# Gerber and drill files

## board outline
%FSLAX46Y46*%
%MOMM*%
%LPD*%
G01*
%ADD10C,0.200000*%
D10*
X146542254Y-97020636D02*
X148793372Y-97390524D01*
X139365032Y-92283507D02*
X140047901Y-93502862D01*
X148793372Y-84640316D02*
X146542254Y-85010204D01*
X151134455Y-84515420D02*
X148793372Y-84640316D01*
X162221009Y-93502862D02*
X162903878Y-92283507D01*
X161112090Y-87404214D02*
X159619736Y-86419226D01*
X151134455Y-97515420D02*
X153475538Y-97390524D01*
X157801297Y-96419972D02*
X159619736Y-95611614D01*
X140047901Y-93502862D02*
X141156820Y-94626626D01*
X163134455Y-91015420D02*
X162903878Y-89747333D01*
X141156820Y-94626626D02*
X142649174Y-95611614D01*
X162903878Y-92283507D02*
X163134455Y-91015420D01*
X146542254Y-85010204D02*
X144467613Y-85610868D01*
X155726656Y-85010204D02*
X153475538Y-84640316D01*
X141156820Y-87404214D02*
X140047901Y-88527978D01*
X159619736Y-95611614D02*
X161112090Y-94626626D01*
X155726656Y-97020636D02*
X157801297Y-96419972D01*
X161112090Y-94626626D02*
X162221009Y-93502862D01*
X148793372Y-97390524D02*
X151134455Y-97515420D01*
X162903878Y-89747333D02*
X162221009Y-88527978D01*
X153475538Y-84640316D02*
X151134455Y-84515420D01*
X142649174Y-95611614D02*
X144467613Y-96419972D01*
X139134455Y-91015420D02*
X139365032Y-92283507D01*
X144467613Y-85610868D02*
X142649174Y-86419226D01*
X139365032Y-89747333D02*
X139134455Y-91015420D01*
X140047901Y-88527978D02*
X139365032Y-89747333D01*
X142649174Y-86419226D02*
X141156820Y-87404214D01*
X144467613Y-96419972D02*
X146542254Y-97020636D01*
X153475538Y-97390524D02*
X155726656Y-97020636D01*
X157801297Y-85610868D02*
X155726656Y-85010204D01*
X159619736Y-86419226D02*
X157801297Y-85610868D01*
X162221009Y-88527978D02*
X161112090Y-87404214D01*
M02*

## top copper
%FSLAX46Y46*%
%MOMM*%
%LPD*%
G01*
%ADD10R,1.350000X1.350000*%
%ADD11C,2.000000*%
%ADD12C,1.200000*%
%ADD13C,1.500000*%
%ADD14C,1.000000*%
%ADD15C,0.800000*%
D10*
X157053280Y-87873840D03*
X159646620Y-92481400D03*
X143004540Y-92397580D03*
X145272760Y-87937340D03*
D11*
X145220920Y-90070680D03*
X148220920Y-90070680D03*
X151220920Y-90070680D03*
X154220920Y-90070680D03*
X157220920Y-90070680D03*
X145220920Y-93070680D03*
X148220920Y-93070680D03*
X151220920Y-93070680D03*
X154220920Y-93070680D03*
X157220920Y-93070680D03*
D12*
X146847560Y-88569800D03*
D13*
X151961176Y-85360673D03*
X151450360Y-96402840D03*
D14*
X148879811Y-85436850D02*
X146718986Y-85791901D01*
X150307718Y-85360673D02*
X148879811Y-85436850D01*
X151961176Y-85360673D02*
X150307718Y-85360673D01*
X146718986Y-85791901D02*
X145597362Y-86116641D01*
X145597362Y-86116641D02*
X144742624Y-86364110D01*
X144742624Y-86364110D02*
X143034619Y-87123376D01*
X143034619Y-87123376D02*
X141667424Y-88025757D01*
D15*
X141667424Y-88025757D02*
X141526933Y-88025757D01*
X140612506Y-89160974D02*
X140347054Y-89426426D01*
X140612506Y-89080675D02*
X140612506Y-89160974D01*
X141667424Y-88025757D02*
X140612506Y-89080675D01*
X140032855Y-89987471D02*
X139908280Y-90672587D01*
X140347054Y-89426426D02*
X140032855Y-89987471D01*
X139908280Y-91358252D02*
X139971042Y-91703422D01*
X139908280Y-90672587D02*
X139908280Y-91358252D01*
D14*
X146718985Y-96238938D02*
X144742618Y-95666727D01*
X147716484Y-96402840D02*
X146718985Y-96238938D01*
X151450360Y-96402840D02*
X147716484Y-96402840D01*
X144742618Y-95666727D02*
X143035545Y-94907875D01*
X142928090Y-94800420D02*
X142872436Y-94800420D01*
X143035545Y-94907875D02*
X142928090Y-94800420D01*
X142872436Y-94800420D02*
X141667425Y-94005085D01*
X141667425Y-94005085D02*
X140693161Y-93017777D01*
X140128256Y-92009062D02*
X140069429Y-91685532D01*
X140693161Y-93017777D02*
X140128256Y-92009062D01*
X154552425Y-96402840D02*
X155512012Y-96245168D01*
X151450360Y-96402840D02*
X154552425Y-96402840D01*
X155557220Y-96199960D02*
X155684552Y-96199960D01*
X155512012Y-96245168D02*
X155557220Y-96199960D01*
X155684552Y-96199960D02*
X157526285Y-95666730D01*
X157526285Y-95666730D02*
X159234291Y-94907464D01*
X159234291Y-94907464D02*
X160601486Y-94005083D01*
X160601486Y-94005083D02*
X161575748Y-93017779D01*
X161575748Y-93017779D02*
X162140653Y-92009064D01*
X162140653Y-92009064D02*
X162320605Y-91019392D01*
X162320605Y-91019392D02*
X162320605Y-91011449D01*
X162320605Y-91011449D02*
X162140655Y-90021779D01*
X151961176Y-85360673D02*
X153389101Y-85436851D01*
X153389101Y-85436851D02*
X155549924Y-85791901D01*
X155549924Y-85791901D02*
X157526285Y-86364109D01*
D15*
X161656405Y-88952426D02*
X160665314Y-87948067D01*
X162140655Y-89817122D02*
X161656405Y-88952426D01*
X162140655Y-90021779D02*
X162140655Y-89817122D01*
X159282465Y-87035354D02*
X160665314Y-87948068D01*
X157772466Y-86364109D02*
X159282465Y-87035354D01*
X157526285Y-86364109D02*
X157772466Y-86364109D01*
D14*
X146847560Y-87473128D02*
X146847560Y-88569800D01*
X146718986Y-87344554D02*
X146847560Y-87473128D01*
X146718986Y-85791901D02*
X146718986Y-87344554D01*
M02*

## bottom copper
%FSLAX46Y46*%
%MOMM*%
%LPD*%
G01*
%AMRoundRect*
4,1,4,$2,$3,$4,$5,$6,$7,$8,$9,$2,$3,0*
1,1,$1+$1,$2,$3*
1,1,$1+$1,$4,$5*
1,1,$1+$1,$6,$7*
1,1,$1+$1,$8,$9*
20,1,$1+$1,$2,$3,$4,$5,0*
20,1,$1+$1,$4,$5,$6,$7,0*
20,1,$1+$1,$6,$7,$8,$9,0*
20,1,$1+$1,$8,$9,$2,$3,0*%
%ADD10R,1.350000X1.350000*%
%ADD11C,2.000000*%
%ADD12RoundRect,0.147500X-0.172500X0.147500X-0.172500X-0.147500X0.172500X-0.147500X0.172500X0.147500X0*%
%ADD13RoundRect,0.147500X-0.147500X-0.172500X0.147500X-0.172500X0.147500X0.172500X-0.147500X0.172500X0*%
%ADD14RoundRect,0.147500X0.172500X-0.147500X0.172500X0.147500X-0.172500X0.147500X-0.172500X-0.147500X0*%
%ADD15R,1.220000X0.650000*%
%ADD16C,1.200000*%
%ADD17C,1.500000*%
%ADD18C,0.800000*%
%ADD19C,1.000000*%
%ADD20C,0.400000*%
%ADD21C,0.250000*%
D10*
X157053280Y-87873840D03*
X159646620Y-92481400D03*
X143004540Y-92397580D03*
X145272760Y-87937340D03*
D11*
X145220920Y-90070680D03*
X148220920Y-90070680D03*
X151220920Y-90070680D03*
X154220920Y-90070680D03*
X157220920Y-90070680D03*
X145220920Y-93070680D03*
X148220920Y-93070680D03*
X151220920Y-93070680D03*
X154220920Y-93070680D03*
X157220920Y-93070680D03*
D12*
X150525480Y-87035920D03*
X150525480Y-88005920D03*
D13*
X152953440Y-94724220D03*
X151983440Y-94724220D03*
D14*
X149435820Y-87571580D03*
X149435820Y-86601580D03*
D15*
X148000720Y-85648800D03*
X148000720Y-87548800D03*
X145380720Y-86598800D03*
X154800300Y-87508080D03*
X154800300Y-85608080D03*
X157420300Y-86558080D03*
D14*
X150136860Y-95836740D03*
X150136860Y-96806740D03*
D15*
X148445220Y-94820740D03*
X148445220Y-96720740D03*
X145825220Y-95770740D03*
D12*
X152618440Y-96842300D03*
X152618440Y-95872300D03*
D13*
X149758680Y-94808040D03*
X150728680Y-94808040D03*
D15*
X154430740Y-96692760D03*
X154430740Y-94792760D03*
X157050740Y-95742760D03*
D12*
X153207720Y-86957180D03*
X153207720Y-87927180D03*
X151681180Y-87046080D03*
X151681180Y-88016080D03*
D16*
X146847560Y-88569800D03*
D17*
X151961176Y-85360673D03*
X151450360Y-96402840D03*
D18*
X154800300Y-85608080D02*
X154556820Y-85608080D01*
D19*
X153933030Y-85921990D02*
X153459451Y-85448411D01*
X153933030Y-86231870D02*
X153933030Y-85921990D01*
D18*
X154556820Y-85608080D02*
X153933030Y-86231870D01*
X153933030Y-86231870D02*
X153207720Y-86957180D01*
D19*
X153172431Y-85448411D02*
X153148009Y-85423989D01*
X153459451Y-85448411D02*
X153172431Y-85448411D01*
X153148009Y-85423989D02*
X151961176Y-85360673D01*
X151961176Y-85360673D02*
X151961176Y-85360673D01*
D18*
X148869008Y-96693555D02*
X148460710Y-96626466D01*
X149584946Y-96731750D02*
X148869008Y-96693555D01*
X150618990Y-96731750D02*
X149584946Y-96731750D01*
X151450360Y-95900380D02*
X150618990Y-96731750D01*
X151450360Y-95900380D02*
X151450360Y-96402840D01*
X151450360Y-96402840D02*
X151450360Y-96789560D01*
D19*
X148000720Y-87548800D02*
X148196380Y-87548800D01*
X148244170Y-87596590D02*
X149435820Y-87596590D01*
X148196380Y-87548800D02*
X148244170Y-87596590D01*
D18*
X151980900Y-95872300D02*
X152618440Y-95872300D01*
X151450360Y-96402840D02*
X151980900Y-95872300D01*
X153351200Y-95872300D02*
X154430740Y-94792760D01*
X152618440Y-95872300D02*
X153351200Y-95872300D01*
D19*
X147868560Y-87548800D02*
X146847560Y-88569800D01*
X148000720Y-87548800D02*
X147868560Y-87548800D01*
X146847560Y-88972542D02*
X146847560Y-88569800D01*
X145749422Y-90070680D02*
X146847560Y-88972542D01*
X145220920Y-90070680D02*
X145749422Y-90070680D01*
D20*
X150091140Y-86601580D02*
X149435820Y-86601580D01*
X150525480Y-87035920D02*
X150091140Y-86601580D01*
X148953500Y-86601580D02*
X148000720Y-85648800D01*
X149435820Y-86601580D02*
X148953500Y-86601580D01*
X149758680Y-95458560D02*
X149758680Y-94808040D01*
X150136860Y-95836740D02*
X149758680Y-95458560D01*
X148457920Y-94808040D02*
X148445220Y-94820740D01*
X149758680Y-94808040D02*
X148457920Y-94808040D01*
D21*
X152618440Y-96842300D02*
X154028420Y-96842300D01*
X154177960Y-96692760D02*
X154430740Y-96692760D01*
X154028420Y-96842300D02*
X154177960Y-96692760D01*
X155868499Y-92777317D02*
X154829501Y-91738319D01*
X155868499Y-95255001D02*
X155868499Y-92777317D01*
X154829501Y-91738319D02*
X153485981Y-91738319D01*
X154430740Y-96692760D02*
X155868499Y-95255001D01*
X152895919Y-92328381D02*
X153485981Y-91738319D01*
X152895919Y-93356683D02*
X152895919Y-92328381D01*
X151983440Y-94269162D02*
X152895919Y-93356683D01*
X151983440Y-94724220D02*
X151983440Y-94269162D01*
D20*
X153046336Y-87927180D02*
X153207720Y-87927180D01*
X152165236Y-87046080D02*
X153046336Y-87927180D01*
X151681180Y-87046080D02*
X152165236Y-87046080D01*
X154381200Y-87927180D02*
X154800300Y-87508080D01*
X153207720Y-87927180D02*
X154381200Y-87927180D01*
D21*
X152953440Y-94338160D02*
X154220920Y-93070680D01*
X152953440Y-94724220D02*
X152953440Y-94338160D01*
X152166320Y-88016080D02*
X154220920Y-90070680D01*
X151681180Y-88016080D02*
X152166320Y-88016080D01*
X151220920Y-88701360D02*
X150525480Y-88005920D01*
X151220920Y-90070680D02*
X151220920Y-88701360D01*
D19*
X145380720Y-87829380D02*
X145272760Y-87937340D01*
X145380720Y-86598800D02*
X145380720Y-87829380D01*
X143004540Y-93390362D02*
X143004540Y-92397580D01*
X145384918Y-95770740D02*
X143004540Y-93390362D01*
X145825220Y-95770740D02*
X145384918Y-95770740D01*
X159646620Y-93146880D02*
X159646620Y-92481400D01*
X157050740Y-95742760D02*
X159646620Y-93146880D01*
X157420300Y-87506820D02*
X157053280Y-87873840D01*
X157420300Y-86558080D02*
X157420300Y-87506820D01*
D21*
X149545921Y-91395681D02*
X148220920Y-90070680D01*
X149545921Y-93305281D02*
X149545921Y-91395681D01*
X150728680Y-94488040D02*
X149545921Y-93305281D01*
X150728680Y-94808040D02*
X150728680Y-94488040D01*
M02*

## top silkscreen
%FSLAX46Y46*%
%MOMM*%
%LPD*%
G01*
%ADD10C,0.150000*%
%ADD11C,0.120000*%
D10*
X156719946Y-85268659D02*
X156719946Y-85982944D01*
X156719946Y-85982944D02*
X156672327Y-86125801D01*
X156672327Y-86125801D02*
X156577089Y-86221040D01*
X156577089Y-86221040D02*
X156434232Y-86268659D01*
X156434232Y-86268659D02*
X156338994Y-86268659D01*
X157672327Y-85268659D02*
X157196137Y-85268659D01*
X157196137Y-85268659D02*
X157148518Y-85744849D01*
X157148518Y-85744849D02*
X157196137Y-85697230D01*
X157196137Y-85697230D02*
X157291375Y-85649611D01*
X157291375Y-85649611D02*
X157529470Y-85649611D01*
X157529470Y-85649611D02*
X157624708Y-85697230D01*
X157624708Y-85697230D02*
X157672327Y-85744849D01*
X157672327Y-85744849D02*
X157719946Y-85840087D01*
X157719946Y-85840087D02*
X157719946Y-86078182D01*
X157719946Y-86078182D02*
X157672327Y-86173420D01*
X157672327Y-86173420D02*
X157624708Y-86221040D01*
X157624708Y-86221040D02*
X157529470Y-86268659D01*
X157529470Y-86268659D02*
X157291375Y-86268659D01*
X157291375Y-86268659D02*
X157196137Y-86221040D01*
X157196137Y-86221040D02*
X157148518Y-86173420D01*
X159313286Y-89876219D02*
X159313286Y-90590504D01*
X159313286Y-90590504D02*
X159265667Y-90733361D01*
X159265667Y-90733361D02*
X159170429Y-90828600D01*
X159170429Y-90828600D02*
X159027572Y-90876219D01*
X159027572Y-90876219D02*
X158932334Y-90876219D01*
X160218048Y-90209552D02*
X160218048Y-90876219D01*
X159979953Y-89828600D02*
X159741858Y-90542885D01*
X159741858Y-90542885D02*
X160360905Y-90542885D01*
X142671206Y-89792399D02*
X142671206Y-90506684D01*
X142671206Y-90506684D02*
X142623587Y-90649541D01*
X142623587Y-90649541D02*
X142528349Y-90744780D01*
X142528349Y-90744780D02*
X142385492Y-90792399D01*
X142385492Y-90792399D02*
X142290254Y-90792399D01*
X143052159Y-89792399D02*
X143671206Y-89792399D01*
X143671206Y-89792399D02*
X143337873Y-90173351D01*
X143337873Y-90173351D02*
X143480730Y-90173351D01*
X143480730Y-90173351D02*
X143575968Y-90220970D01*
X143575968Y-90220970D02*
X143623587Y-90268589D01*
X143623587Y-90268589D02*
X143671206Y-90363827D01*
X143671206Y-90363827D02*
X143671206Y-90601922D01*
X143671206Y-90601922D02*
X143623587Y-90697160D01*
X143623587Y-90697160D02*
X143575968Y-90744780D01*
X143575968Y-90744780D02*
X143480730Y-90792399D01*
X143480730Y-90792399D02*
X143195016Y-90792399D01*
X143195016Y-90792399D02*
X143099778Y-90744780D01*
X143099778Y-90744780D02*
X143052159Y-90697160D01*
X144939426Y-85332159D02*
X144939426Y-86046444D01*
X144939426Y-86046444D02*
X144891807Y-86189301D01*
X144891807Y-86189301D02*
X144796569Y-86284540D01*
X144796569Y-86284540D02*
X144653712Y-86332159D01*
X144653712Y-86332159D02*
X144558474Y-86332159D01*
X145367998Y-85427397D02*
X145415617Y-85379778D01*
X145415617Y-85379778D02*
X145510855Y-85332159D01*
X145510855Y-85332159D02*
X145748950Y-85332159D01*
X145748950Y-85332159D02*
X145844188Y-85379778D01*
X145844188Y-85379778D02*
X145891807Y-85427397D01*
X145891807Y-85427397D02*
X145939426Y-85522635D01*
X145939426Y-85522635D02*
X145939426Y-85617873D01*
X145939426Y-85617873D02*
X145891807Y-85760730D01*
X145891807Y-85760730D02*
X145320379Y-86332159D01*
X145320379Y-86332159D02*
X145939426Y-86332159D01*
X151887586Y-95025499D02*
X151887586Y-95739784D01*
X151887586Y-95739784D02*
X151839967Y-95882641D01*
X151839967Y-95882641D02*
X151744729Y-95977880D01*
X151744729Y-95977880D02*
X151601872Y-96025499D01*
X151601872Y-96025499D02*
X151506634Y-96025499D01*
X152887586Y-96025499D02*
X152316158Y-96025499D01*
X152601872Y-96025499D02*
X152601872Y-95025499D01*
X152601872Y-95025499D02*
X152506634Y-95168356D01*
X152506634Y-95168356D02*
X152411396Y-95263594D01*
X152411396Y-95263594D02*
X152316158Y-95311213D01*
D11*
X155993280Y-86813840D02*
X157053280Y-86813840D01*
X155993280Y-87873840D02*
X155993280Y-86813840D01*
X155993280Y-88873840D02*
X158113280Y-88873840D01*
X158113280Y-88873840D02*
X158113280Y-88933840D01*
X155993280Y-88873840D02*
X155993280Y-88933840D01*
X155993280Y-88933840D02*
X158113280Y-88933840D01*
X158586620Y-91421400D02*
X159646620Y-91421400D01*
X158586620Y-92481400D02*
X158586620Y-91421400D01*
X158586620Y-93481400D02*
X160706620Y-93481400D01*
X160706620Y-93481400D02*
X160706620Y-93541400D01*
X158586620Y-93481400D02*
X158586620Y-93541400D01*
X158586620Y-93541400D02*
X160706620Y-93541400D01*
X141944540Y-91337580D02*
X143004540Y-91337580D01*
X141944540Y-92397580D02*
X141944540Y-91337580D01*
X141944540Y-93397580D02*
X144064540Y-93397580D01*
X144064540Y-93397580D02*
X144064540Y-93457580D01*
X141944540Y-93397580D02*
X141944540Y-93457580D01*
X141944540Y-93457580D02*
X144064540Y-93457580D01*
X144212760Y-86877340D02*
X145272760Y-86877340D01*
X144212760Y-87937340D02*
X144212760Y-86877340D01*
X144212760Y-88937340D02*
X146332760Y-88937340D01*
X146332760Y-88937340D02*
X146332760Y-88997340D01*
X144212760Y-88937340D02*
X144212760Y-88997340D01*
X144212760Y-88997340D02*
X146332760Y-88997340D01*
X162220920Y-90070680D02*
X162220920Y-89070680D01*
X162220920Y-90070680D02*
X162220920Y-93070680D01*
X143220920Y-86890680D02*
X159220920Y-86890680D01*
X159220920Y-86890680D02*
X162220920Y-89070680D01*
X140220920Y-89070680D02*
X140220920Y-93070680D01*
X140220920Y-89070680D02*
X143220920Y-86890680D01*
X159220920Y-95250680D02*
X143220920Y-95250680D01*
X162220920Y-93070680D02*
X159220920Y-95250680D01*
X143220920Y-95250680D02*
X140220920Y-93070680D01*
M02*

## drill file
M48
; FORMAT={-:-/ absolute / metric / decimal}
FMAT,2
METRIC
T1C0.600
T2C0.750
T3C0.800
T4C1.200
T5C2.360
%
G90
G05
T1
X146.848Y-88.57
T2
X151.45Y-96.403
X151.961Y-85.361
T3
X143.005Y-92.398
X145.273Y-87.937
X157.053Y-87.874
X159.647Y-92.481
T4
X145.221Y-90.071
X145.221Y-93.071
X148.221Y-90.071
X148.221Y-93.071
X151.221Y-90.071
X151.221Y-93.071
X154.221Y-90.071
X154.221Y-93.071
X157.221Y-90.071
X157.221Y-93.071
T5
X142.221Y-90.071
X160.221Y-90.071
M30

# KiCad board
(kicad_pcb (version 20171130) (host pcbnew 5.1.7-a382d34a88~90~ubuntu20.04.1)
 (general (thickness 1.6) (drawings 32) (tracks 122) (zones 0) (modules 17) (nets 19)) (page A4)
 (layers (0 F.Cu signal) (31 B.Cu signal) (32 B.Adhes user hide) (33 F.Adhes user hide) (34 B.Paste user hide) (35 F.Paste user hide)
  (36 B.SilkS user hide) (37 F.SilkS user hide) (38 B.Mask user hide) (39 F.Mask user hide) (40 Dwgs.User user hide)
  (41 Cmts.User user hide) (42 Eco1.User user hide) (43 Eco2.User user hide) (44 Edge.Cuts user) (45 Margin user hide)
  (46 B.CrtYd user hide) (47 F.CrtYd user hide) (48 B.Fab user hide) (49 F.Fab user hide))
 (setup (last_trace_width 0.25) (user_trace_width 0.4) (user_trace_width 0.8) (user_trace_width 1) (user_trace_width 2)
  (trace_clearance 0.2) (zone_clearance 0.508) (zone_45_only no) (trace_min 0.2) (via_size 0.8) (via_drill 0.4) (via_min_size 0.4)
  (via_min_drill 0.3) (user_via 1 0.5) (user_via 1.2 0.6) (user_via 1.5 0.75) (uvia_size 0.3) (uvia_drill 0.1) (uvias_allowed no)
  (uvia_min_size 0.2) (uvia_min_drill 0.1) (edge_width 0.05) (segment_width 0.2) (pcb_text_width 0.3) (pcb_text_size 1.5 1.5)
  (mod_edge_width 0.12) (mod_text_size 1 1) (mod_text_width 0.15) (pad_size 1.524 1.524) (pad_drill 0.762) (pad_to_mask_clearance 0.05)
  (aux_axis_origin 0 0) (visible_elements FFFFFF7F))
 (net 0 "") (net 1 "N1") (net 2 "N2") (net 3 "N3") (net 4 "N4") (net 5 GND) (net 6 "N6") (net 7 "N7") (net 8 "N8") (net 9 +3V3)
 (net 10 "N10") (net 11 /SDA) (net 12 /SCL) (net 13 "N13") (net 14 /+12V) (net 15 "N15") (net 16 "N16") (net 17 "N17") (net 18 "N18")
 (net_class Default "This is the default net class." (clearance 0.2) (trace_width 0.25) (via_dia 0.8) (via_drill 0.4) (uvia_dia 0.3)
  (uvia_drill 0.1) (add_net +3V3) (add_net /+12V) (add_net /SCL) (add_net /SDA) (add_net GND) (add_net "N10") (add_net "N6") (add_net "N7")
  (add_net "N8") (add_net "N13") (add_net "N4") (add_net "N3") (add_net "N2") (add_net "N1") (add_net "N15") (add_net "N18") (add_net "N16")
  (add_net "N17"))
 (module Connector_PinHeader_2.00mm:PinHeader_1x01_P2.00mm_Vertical (layer F.Cu) (at 157.05328 87.87384)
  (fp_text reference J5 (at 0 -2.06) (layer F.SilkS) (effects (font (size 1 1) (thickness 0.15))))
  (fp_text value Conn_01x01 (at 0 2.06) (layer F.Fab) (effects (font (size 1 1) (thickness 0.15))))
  (fp_line (start -1.06 -1.06) (end 0 -1.06) (layer F.SilkS) (width 0.12))
  (fp_line (start -1.06 0) (end -1.06 -1.06) (layer F.SilkS) (width 0.12))
  (fp_line (start -1.06 1) (end 1.06 1) (layer F.SilkS) (width 0.12))
  (fp_line (start 1.06 1) (end 1.06 1.06) (layer F.SilkS) (width 0.12))
  (fp_line (start -1.06 1) (end -1.06 1.06) (layer F.SilkS) (width 0.12))
  (fp_line (start -1.06 1.06) (end 1.06 1.06) (layer F.SilkS) (width 0.12))
  (pad 1 thru_hole rect (at 0 0) (size 1.35 1.35) (drill 0.8) (layers *.Cu *.Mask) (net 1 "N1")))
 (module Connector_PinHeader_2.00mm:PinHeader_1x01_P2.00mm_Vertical (layer F.Cu) (at 159.64662 92.4814)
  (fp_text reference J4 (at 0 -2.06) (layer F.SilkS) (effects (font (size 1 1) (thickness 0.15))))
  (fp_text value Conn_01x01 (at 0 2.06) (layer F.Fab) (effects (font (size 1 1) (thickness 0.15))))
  (fp_line (start -1.06 -1.06) (end 0 -1.06) (layer F.SilkS) (width 0.12))
  (fp_line (start -1.06 0) (end -1.06 -1.06) (layer F.SilkS) (width 0.12))
  (fp_line (start -1.06 1) (end 1.06 1) (layer F.SilkS) (width 0.12))
  (fp_line (start 1.06 1) (end 1.06 1.06) (layer F.SilkS) (width 0.12))
  (fp_line (start -1.06 1) (end -1.06 1.06) (layer F.SilkS) (width 0.12))
  (fp_line (start -1.06 1.06) (end 1.06 1.06) (layer F.SilkS) (width 0.12))
  (pad 1 thru_hole rect (at 0 0) (size 1.35 1.35) (drill 0.8) (layers *.Cu *.Mask) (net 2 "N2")))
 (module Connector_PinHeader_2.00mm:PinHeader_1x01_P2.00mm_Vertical (layer F.Cu) (at 143.00454 92.39758)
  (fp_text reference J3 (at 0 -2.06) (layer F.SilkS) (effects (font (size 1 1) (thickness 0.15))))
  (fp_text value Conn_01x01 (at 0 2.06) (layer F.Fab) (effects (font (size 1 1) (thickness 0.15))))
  (fp_line (start -1.06 -1.06) (end 0 -1.06) (layer F.SilkS) (width 0.12))
  (fp_line (start -1.06 0) (end -1.06 -1.06) (layer F.SilkS) (width 0.12))
  (fp_line (start -1.06 1) (end 1.06 1) (layer F.SilkS) (width 0.12))
  (fp_line (start 1.06 1) (end 1.06 1.06) (layer F.SilkS) (width 0.12))
  (fp_line (start -1.06 1) (end -1.06 1.06) (layer F.SilkS) (width 0.12))
  (fp_line (start -1.06 1.06) (end 1.06 1.06) (layer F.SilkS) (width 0.12))
  (pad 1 thru_hole rect (at 0 0) (size 1.35 1.35) (drill 0.8) (layers *.Cu *.Mask) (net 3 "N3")))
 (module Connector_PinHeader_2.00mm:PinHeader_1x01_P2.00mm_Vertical (layer F.Cu) (at 145.27276 87.93734)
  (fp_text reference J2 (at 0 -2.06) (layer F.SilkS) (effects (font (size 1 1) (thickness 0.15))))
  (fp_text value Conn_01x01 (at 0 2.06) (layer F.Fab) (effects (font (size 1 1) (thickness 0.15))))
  (fp_line (start -1.06 -1.06) (end 0 -1.06) (layer F.SilkS) (width 0.12))
  (fp_line (start -1.06 0) (end -1.06 -1.06) (layer F.SilkS) (width 0.12))
  (fp_line (start -1.06 1) (end 1.06 1) (layer F.SilkS) (width 0.12))
  (fp_line (start 1.06 1) (end 1.06 1.06) (layer F.SilkS) (width 0.12))
  (fp_line (start -1.06 1) (end -1.06 1.06) (layer F.SilkS) (width 0.12))
  (fp_line (start -1.06 1.06) (end 1.06 1.06) (layer F.SilkS) (width 0.12))
  (pad 1 thru_hole rect (at 0 0) (size 1.35 1.35) (drill 0.8) (layers *.Cu *.Mask) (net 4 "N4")))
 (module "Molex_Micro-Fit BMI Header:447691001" (layer F.Cu) (at 152.22092 95.07068)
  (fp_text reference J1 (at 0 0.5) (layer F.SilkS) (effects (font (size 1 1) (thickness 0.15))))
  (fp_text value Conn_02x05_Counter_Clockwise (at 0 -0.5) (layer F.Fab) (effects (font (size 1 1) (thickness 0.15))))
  (fp_line (start 10 -5) (end 10 -6) (layer F.SilkS) (width 0.12))
  (fp_line (start 10 -5) (end 10 -2) (layer F.SilkS) (width 0.12))
  (fp_line (start -9 -8.18) (end 7 -8.18) (layer F.SilkS) (width 0.12))
  (fp_line (start 7 -8.18) (end 10 -6) (layer F.SilkS) (width 0.12))
  (fp_line (start -12 -6) (end -12 -2) (layer F.SilkS) (width 0.12))
  (fp_line (start -12 -6) (end -9 -8.18) (layer F.SilkS) (width 0.12))
  (fp_line (start 7 0.18) (end -9 0.18) (layer F.SilkS) (width 0.12))
  (fp_line (start 10 -2) (end 7 0.18) (layer F.SilkS) (width 0.12))
  (fp_line (start -9 0.18) (end -12 -2) (layer F.SilkS) (width 0.12))
  (pad "" np_thru_hole circle (at -10 -5) (size 2.36 2.36) (drill 2.36) (layers *.Cu *.Mask))
  (pad "" np_thru_hole circle (at 8 -5) (size 2.36 2.36) (drill 2.36) (layers *.Cu *.Mask))
  (pad 1 thru_hole circle (at -7 -5) (size 2 2) (drill 1.2) (layers *.Cu *.Mask) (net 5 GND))
  (pad 3 thru_hole circle (at -4 -5) (size 2 2) (drill 1.2) (layers *.Cu *.Mask) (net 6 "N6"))
  (pad 5 thru_hole circle (at -1 -5) (size 2 2) (drill 1.2) (layers *.Cu *.Mask) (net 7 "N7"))
  (pad 7 thru_hole circle (at 2 -5) (size 2 2) (drill 1.2) (layers *.Cu *.Mask) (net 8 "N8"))
  (pad 9 thru_hole circle (at 5 -5) (size 2 2) (drill 1.2) (layers *.Cu *.Mask) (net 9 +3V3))
  (pad 2 thru_hole circle (at -7 -2) (size 2 2) (drill 1.2) (layers *.Cu *.Mask) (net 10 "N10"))
  (pad 4 thru_hole circle (at -4 -2) (size 2 2) (drill 1.2) (layers *.Cu *.Mask) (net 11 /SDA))
  (pad 6 thru_hole circle (at -1 -2) (size 2 2) (drill 1.2) (layers *.Cu *.Mask) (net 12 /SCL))
  (pad 8 thru_hole circle (at 2 -2) (size 2 2) (drill 1.2) (layers *.Cu *.Mask) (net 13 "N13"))
  (pad 10 thru_hole circle (at 5 -2) (size 2 2) (drill 1.2) (layers *.Cu *.Mask) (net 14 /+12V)))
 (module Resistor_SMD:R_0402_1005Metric (layer B.Cu) (at 150.52548 87.52092 270)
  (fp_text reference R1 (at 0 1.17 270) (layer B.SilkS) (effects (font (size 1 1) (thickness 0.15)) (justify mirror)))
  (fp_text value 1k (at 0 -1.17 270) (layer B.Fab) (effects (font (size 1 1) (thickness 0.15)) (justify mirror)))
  (pad 1 smd roundrect (at -0.485 0 270) (size 0.59 0.64) (layers B.Cu B.Paste B.Mask) (roundrect_rratio 0.25) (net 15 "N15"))
  (pad 2 smd roundrect (at 0.485 0 270) (size 0.59 0.64) (layers B.Cu B.Paste B.Mask) (roundrect_rratio 0.25) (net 7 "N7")))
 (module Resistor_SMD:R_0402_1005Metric (layer B.Cu) (at 152.46844 94.72422)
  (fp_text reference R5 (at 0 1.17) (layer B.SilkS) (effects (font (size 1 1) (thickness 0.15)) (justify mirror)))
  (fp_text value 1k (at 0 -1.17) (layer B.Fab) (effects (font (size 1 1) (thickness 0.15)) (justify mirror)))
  (pad 2 smd roundrect (at 0.485 0) (size 0.59 0.64) (layers B.Cu B.Paste B.Mask) (roundrect_rratio 0.25) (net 13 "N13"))
  (pad 1 smd roundrect (at -0.485 0) (size 0.59 0.64) (layers B.Cu B.Paste B.Mask) (roundrect_rratio 0.25) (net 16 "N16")))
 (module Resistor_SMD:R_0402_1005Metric (layer B.Cu) (at 149.43582 87.08658 90)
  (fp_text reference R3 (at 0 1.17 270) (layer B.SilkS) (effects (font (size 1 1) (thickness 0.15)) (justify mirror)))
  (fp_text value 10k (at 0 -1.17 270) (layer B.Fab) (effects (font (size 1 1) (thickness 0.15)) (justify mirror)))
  (pad 1 smd roundrect (at -0.485 0 90) (size 0.59 0.64) (layers B.Cu B.Paste B.Mask) (roundrect_rratio 0.25) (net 5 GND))
  (pad 2 smd roundrect (at 0.485 0 90) (size 0.59 0.64) (layers B.Cu B.Paste B.Mask) (roundrect_rratio 0.25) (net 15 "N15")))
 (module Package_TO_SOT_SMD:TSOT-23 (layer B.Cu) (at 146.69072 86.5988 180)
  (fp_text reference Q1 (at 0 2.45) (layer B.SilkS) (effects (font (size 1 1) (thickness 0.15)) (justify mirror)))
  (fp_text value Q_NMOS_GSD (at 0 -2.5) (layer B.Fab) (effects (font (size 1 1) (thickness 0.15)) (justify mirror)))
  (pad 1 smd rect (at -1.31 0.95 180) (size 1.22 0.65) (layers B.Cu B.Paste B.Mask) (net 15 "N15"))
  (pad 2 smd rect (at -1.31 -0.95 180) (size 1.22 0.65) (layers B.Cu B.Paste B.Mask) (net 5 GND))
  (pad 3 smd rect (at 1.31 0 180) (size 1.22 0.65) (layers B.Cu B.Paste B.Mask) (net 4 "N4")))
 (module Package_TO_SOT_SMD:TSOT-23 (layer B.Cu) (at 156.1103 86.55808)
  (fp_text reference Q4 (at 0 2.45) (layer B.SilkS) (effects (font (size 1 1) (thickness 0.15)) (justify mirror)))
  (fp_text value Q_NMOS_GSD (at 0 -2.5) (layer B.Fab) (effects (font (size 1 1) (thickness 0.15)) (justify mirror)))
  (pad 1 smd rect (at -1.31 0.95) (size 1.22 0.65) (layers B.Cu B.Paste B.Mask) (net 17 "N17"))
  (pad 2 smd rect (at -1.31 -0.95) (size 1.22 0.65) (layers B.Cu B.Paste B.Mask) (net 5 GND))
  (pad 3 smd rect (at 1.31 0) (size 1.22 0.65) (layers B.Cu B.Paste B.Mask) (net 1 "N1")))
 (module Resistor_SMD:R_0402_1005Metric (layer B.Cu) (at 150.13686 96.32174 90)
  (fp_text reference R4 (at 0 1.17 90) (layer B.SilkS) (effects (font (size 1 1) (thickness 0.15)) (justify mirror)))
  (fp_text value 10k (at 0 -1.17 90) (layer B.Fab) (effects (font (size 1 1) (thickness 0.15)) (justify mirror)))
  (pad 2 smd roundrect (at 0.485 0 90) (size 0.59 0.64) (layers B.Cu B.Paste B.Mask) (roundrect_rratio 0.25) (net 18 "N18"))
  (pad 1 smd roundrect (at -0.485 0 90) (size 0.59 0.64) (layers B.Cu B.Paste B.Mask) (roundrect_rratio 0.25) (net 5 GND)))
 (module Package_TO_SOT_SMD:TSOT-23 (layer B.Cu) (at 147.13522 95.77074 180)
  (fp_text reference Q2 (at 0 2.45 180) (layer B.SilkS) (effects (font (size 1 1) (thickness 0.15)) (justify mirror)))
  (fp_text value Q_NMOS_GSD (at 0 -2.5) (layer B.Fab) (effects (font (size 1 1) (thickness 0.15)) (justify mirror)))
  (pad 1 smd rect (at -1.31 0.95 180) (size 1.22 0.65) (layers B.Cu B.Paste B.Mask) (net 18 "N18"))
  (pad 2 smd rect (at -1.31 -0.95 180) (size 1.22 0.65) (layers B.Cu B.Paste B.Mask) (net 5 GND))
  (pad 3 smd rect (at 1.31 0 180) (size 1.22 0.65) (layers B.Cu B.Paste B.Mask) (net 3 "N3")))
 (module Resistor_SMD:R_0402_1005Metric (layer B.Cu) (at 152.61844 96.3573 270)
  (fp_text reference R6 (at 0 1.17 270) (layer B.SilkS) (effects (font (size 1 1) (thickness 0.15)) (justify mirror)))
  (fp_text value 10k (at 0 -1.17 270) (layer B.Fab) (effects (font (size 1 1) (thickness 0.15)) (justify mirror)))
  (pad 2 smd roundrect (at 0.485 0 270) (size 0.59 0.64) (layers B.Cu B.Paste B.Mask) (roundrect_rratio 0.25) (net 16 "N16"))
  (pad 1 smd roundrect (at -0.485 0 270) (size 0.59 0.64) (layers B.Cu B.Paste B.Mask) (roundrect_rratio 0.25) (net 5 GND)))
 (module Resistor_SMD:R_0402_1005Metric (layer B.Cu) (at 150.24368 94.80804)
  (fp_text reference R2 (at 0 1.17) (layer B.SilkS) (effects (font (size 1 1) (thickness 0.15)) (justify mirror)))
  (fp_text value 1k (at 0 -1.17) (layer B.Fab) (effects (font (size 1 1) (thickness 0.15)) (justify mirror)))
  (pad 1 smd roundrect (at -0.485 0) (size 0.59 0.64) (layers B.Cu B.Paste B.Mask) (roundrect_rratio 0.25) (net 18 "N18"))
  (pad 2 smd roundrect (at 0.485 0) (size 0.59 0.64) (layers B.Cu B.Paste B.Mask) (roundrect_rratio 0.25) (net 6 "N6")))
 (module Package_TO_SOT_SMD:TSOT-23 (layer B.Cu) (at 155.74074 95.74276)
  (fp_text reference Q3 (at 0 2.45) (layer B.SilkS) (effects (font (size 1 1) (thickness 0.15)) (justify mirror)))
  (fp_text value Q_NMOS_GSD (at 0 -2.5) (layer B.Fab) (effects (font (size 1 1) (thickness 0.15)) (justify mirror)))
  (pad 1 smd rect (at -1.31 0.95) (size 1.22 0.65) (layers B.Cu B.Paste B.Mask) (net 16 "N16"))
  (pad 2 smd rect (at -1.31 -0.95) (size 1.22 0.65) (layers B.Cu B.Paste B.Mask) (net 5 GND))
  (pad 3 smd rect (at 1.31 0) (size 1.22 0.65) (layers B.Cu B.Paste B.Mask) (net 2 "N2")))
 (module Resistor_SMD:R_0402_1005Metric (layer B.Cu) (at 153.20772 87.44218 270)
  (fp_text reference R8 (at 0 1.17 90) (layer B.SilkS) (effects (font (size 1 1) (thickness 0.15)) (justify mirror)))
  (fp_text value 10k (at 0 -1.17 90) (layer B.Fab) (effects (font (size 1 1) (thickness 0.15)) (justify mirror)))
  (pad 1 smd roundrect (at -0.485 0 270) (size 0.59 0.64) (layers B.Cu B.Paste B.Mask) (roundrect_rratio 0.25) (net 5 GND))
  (pad 2 smd roundrect (at 0.485 0 270) (size 0.59 0.64) (layers B.Cu B.Paste B.Mask) (roundrect_rratio 0.25) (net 17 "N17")))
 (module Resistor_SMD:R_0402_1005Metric (layer B.Cu) (at 151.68118 87.53108 270)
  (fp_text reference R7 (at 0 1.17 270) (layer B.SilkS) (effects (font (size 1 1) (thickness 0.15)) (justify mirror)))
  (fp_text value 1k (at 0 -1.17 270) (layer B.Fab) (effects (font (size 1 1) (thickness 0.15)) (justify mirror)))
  (pad 1 smd roundrect (at -0.485 0 270) (size 0.59 0.64) (layers B.Cu B.Paste B.Mask) (roundrect_rratio 0.25) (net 17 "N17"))
  (pad 2 smd roundrect (at 0.485 0 270) (size 0.59 0.64) (layers B.Cu B.Paste B.Mask) (roundrect_rratio 0.25) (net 8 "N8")))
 (gr_line (start 146.542254 97.020636) (end 148.793372 97.390524) (layer Edge.Cuts) (width 0.2))
 (gr_line (start 139.365032 92.283507) (end 140.047901 93.502862) (layer Edge.Cuts) (width 0.2))
 (gr_line (start 148.793372 84.640316) (end 146.542254 85.010204) (layer Edge.Cuts) (width 0.2))
 (gr_line (start 151.134455 84.51542) (end 148.793372 84.640316) (layer Edge.Cuts) (width 0.2))
 (gr_line (start 162.221009 93.502862) (end 162.903878 92.283507) (layer Edge.Cuts) (width 0.2))
 (gr_line (start 161.11209 87.404214) (end 159.619736 86.419226) (layer Edge.Cuts) (width 0.2))
 (gr_line (start 151.134455 97.51542) (end 153.475538 97.390524) (layer Edge.Cuts) (width 0.2))
 (gr_line (start 157.801297 96.419972) (end 159.619736 95.611614) (layer Edge.Cuts) (width 0.2))
 (gr_line (start 140.047901 93.502862) (end 141.15682 94.626626) (layer Edge.Cuts) (width 0.2))
 (gr_line (start 163.134455 91.01542) (end 162.903878 89.747333) (layer Edge.Cuts) (width 0.2))
 (gr_line (start 141.15682 94.626626) (end 142.649174 95.611614) (layer Edge.Cuts) (width 0.2))
 (gr_line (start 162.903878 92.283507) (end 163.134455 91.01542) (layer Edge.Cuts) (width 0.2))
 (gr_line (start 146.542254 85.010204) (end 144.467613 85.610868) (layer Edge.Cuts) (width 0.2))
 (gr_line (start 155.726656 85.010204) (end 153.475538 84.640316) (layer Edge.Cuts) (width 0.2))
 (gr_line (start 141.15682 87.404214) (end 140.047901 88.527978) (layer Edge.Cuts) (width 0.2))
 (gr_line (start 159.619736 95.611614) (end 161.11209 94.626626) (layer Edge.Cuts) (width 0.2))
 (gr_line (start 155.726656 97.020636) (end 157.801297 96.419972) (layer Edge.Cuts) (width 0.2))
 (gr_line (start 161.11209 94.626626) (end 162.221009 93.502862) (layer Edge.Cuts) (width 0.2))
 (gr_line (start 148.793372 97.390524) (end 151.134455 97.51542) (layer Edge.Cuts) (width 0.2))
 (gr_line (start 162.903878 89.747333) (end 162.221009 88.527978) (layer Edge.Cuts) (width 0.2))
 (gr_line (start 153.475538 84.640316) (end 151.134455 84.51542) (layer Edge.Cuts) (width 0.2))
 (gr_line (start 142.649174 95.611614) (end 144.467613 96.419972) (layer Edge.Cuts) (width 0.2))
 (gr_line (start 139.134455 91.01542) (end 139.365032 92.283507) (layer Edge.Cuts) (width 0.2))
 (gr_line (start 144.467613 85.610868) (end 142.649174 86.419226) (layer Edge.Cuts) (width 0.2))
 (gr_line (start 139.365032 89.747333) (end 139.134455 91.01542) (layer Edge.Cuts) (width 0.2))
 (gr_line (start 140.047901 88.527978) (end 139.365032 89.747333) (layer Edge.Cuts) (width 0.2))
 (gr_line (start 142.649174 86.419226) (end 141.15682 87.404214) (layer Edge.Cuts) (width 0.2))
 (gr_line (start 144.467613 96.419972) (end 146.542254 97.020636) (layer Edge.Cuts) (width 0.2))
 (gr_line (start 153.475538 97.390524) (end 155.726656 97.020636) (layer Edge.Cuts) (width 0.2))
 (gr_line (start 157.801297 85.610868) (end 155.726656 85.010204) (layer Edge.Cuts) (width 0.2))
 (gr_line (start 159.619736 86.419226) (end 157.801297 85.610868) (layer Edge.Cuts) (width 0.2))
 (gr_line (start 162.221009 88.527978) (end 161.11209 87.404214) (layer Edge.Cuts) (width 0.2))
 (via (at 146.84756 88.5698) (size 1.2) (drill 0.6) (layers F.Cu B.Cu) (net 5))
 (segment (start 154.8003 85.60808) (end 154.55682 85.60808) (width 0.8) (layer B.Cu) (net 5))
 (segment (start 153.93303 85.92199) (end 153.459451 85.448411) (width 1) (layer B.Cu) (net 5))
 (segment (start 153.93303 86.23187) (end 153.93303 85.92199) (width 1) (layer B.Cu) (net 5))
 (segment (start 154.55682 85.60808) (end 153.93303 86.23187) (width 0.8) (layer B.Cu) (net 5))
 (segment (start 153.93303 86.23187) (end 153.20772 86.95718) (width 0.8) (layer B.Cu) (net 5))
 (segment (start 153.172431 85.448411) (end 153.148009 85.423989) (width 1) (layer B.Cu) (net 5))
 (segment (start 153.459451 85.448411) (end 153.172431 85.448411) (width 1) (layer B.Cu) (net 5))
 (segment (start 153.148009 85.423989) (end 151.961176 85.360673) (width 1) (layer B.Cu) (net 5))
 (segment (start 151.961176 85.360673) (end 151.961176 85.360673) (width 1) (layer B.Cu) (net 5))
 (via (at 151.961176 85.360673) (size 1.5) (drill 0.75) (layers F.Cu B.Cu) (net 5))
 (segment (start 148.879811 85.43685) (end 146.718986 85.791901) (width 1) (layer F.Cu) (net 5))
 (segment (start 150.307718 85.360673) (end 148.879811 85.43685) (width 1) (layer F.Cu) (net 5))
 (segment (start 151.961176 85.360673) (end 150.307718 85.360673) (width 1) (layer F.Cu) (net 5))
 (segment (start 146.718986 85.791901) (end 145.597362 86.116641) (width 1) (layer F.Cu) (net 5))
 (segment (start 145.597362 86.116641) (end 144.742624 86.36411) (width 1) (layer F.Cu) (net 5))
 (segment (start 144.742624 86.36411) (end 143.034619 87.123376) (width 1) (layer F.Cu) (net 5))
 (segment (start 143.034619 87.123376) (end 141.667424 88.025757) (width 1) (layer F.Cu) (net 5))
 (segment (start 141.667424 88.025757) (end 141.526933 88.025757) (width 0.8) (layer F.Cu) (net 5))
 (segment (start 140.612506 89.160974) (end 140.347054 89.426426) (width 0.8) (layer F.Cu) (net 5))
 (segment (start 140.612506 89.080675) (end 140.612506 89.160974) (width 0.8) (layer F.Cu) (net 5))
 (segment (start 141.667424 88.025757) (end 140.612506 89.080675) (width 0.8) (layer F.Cu) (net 5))
 (segment (start 140.032855 89.987471) (end 139.90828 90.672587) (width 0.8) (layer F.Cu) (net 5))
 (segment (start 140.347054 89.426426) (end 140.032855 89.987471) (width 0.8) (layer F.Cu) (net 5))
 (segment (start 139.90828 91.358252) (end 139.971042 91.703422) (width 0.8) (layer F.Cu) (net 5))
 (segment (start 139.90828 90.672587) (end 139.90828 91.358252) (width 0.8) (layer F.Cu) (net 5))
 (segment (start 148.869008 96.693555) (end 148.46071 96.626466) (width 0.8) (layer B.Cu) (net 5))
 (segment (start 149.584946 96.73175) (end 148.869008 96.693555) (width 0.8) (layer B.Cu) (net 5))
 (segment (start 150.61899 96.73175) (end 149.584946 96.73175) (width 0.8) (layer B.Cu) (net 5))
 (segment (start 151.45036 95.90038) (end 150.61899 96.73175) (width 0.8) (layer B.Cu) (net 5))
 (segment (start 151.45036 95.90038) (end 151.45036 96.40284) (width 0.8) (layer B.Cu) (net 5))
 (segment (start 151.45036 96.40284) (end 151.45036 96.78956) (width 0.8) (layer B.Cu) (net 5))
 (via (at 151.45036 96.40284) (size 1.5) (drill 0.75) (layers F.Cu B.Cu) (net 5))
 (segment (start 148.00072 87.5488) (end 148.19638 87.5488) (width 1) (layer B.Cu) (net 5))
 (segment (start 148.24417 87.59659) (end 149.43582 87.59659) (width 1) (layer B.Cu) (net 5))
 (segment (start 148.19638 87.5488) (end 148.24417 87.59659) (width 1) (layer B.Cu) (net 5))
 (segment (start 146.718985 96.238938) (end 144.742618 95.666727) (width 1) (layer F.Cu) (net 5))
 (segment (start 147.716484 96.40284) (end 146.718985 96.238938) (width 1) (layer F.Cu) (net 5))
 (segment (start 151.45036 96.40284) (end 147.716484 96.40284) (width 1) (layer F.Cu) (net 5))
 (segment (start 144.742618 95.666727) (end 143.035545 94.907875) (width 1) (layer F.Cu) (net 5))
 (segment (start 142.92809 94.80042) (end 142.872436 94.80042) (width 1) (layer F.Cu) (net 5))
 (segment (start 143.035545 94.907875) (end 142.92809 94.80042) (width 1) (layer F.Cu) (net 5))
 (segment (start 142.872436 94.80042) (end 141.667425 94.005085) (width 1) (layer F.Cu) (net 5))
 (segment (start 141.667425 94.005085) (end 140.693161 93.017777) (width 1) (layer F.Cu) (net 5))
 (segment (start 140.128256 92.009062) (end 140.069429 91.685532) (width 1) (layer F.Cu) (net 5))
 (segment (start 140.693161 93.017777) (end 140.128256 92.009062) (width 1) (layer F.Cu) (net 5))
 (segment (start 154.552425 96.40284) (end 155.512012 96.245168) (width 1) (layer F.Cu) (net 5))
 (segment (start 151.45036 96.40284) (end 154.552425 96.40284) (width 1) (layer F.Cu) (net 5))
 (segment (start 155.55722 96.19996) (end 155.684552 96.19996) (width 1) (layer F.Cu) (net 5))
 (segment (start 155.512012 96.245168) (end 155.55722 96.19996) (width 1) (layer F.Cu) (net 5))
 (segment (start 155.684552 96.19996) (end 157.526285 95.66673) (width 1) (layer F.Cu) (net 5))
 (segment (start 157.526285 95.66673) (end 159.234291 94.907464) (width 1) (layer F.Cu) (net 5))
 (segment (start 159.234291 94.907464) (end 160.601486 94.005083) (width 1) (layer F.Cu) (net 5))
 (segment (start 160.601486 94.005083) (end 161.575748 93.017779) (width 1) (layer F.Cu) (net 5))
 (segment (start 161.575748 93.017779) (end 162.140653 92.009064) (width 1) (layer F.Cu) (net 5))
 (segment (start 162.140653 92.009064) (end 162.320605 91.019392) (width 1) (layer F.Cu) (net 5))
 (segment (start 162.320605 91.019392) (end 162.320605 91.011449) (width 1) (layer F.Cu) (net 5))
 (segment (start 162.320605 91.011449) (end 162.140655 90.021779) (width 1) (layer F.Cu) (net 5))
 (segment (start 151.961176 85.360673) (end 153.389101 85.436851) (width 1) (layer F.Cu) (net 5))
 (segment (start 153.389101 85.436851) (end 155.549924 85.791901) (width 1) (layer F.Cu) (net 5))
 (segment (start 155.549924 85.791901) (end 157.526285 86.364109) (width 1) (layer F.Cu) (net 5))
 (segment (start 161.656405 88.952426) (end 160.665314 87.948067) (width 0.8) (layer F.Cu) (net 5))
 (segment (start 162.140655 89.817122) (end 161.656405 88.952426) (width 0.8) (layer F.Cu) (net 5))
 (segment (start 162.140655 90.021779) (end 162.140655 89.817122) (width 0.8) (layer F.Cu) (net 5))
 (segment (start 159.282465 87.035354) (end 160.665314 87.948068) (width 0.8) (layer F.Cu) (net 5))
 (segment (start 157.772466 86.364109) (end 159.282465 87.035354) (width 0.8) (layer F.Cu) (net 5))
 (segment (start 157.526285 86.364109) (end 157.772466 86.364109) (width 0.8) (layer F.Cu) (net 5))
 (segment (start 151.9809 95.8723) (end 152.61844 95.8723) (width 0.8) (layer B.Cu) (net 5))
 (segment (start 151.45036 96.40284) (end 151.9809 95.8723) (width 0.8) (layer B.Cu) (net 5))
 (segment (start 153.3512 95.8723) (end 154.43074 94.79276) (width 0.8) (layer B.Cu) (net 5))
 (segment (start 152.61844 95.8723) (end 153.3512 95.8723) (width 0.8) (layer B.Cu) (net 5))
 (segment (start 146.84756 87.473128) (end 146.84756 88.5698) (width 1) (layer F.Cu) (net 5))
 (segment (start 146.718986 87.344554) (end 146.84756 87.473128) (width 1) (layer F.Cu) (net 5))
 (segment (start 146.718986 85.791901) (end 146.718986 87.344554) (width 1) (layer F.Cu) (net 5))
 (segment (start 147.86856 87.5488) (end 146.84756 88.5698) (width 1) (layer B.Cu) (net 5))
 (segment (start 148.00072 87.5488) (end 147.86856 87.5488) (width 1) (layer B.Cu) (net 5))
 (segment (start 146.84756 88.972542) (end 146.84756 88.5698) (width 1) (layer B.Cu) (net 5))
 (segment (start 145.749422 90.07068) (end 146.84756 88.972542) (width 1) (layer B.Cu) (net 5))
 (segment (start 145.22092 90.07068) (end 145.749422 90.07068) (width 1) (layer B.Cu) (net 5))
 (segment (start 150.09114 86.60158) (end 149.43582 86.60158) (width 0.4) (layer B.Cu) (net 15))
 (segment (start 150.52548 87.03592) (end 150.09114 86.60158) (width 0.4) (layer B.Cu) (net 15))
 (segment (start 148.9535 86.60158) (end 148.00072 85.6488) (width 0.4) (layer B.Cu) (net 15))
 (segment (start 149.43582 86.60158) (end 148.9535 86.60158) (width 0.4) (layer B.Cu) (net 15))
 (segment (start 149.75868 95.45856) (end 149.75868 94.80804) (width 0.4) (layer B.Cu) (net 18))
 (segment (start 150.13686 95.83674) (end 149.75868 95.45856) (width 0.4) (layer B.Cu) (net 18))
 (segment (start 148.45792 94.80804) (end 148.44522 94.82074) (width 0.4) (layer B.Cu) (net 18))
 (segment (start 149.75868 94.80804) (end 148.45792 94.80804) (width 0.4) (layer B.Cu) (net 18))
 (segment (start 152.61844 96.8423) (end 154.02842 96.8423) (width 0.25) (layer B.Cu) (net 16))
 (segment (start 154.17796 96.69276) (end 154.43074 96.69276) (width 0.25) (layer B.Cu) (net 16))
 (segment (start 154.02842 96.8423) (end 154.17796 96.69276) (width 0.25) (layer B.Cu) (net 16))
 (segment (start 155.868499 92.777317) (end 154.829501 91.738319) (width 0.25) (layer B.Cu) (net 16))
 (segment (start 155.868499 95.255001) (end 155.868499 92.777317) (width 0.25) (layer B.Cu) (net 16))
 (segment (start 154.829501 91.738319) (end 153.485981 91.738319) (width 0.25) (layer B.Cu) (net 16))
 (segment (start 154.43074 96.69276) (end 155.868499 95.255001) (width 0.25) (layer B.Cu) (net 16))
 (segment (start 152.895919 92.328381) (end 153.485981 91.738319) (width 0.25) (layer B.Cu) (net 16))
 (segment (start 152.895919 93.356683) (end 152.895919 92.328381) (width 0.25) (layer B.Cu) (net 16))
 (segment (start 151.98344 94.269162) (end 152.895919 93.356683) (width 0.25) (layer B.Cu) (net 16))
 (segment (start 151.98344 94.72422) (end 151.98344 94.269162) (width 0.25) (layer B.Cu) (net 16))
 (segment (start 153.046336 87.92718) (end 153.20772 87.92718) (width 0.4) (layer B.Cu) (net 17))
 (segment (start 152.165236 87.04608) (end 153.046336 87.92718) (width 0.4) (layer B.Cu) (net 17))
 (segment (start 151.68118 87.04608) (end 152.165236 87.04608) (width 0.4) (layer B.Cu) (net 17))
 (segment (start 154.3812 87.92718) (end 154.8003 87.50808) (width 0.4) (layer B.Cu) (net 17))
 (segment (start 153.20772 87.92718) (end 154.3812 87.92718) (width 0.4) (layer B.Cu) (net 17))
 (segment (start 152.95344 94.33816) (end 154.22092 93.07068) (width 0.25) (layer B.Cu) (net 13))
 (segment (start 152.95344 94.72422) (end 152.95344 94.33816) (width 0.25) (layer B.Cu) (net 13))
 (segment (start 152.16632 88.01608) (end 154.22092 90.07068) (width 0.25) (layer B.Cu) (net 8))
 (segment (start 151.68118 88.01608) (end 152.16632 88.01608) (width 0.25) (layer B.Cu) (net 8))
 (segment (start 151.22092 88.70136) (end 150.52548 88.00592) (width 0.25) (layer B.Cu) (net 7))
 (segment (start 151.22092 90.07068) (end 151.22092 88.70136) (width 0.25) (layer B.Cu) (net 7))
 (segment (start 145.38072 87.82938) (end 145.27276 87.93734) (width 1) (layer B.Cu) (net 4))
 (segment (start 145.38072 86.5988) (end 145.38072 87.82938) (width 1) (layer B.Cu) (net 4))
 (segment (start 143.00454 93.390362) (end 143.00454 92.39758) (width 1) (layer B.Cu) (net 3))
 (segment (start 145.384918 95.77074) (end 143.00454 93.390362) (width 1) (layer B.Cu) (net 3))
 (segment (start 145.82522 95.77074) (end 145.384918 95.77074) (width 1) (layer B.Cu) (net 3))
 (segment (start 159.64662 93.14688) (end 159.64662 92.4814) (width 1) (layer B.Cu) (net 2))
 (segment (start 157.05074 95.74276) (end 159.64662 93.14688) (width 1) (layer B.Cu) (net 2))
 (segment (start 157.4203 87.50682) (end 157.05328 87.87384) (width 1) (layer B.Cu) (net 1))
 (segment (start 157.4203 86.55808) (end 157.4203 87.50682) (width 1) (layer B.Cu) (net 1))
 (segment (start 149.545921 91.395681) (end 148.22092 90.07068) (width 0.25) (layer B.Cu) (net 6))
 (segment (start 149.545921 93.305281) (end 149.545921 91.395681) (width 0.25) (layer B.Cu) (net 6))
 (segment (start 150.72868 94.48804) (end 149.545921 93.305281) (width 0.25) (layer B.Cu) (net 6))
 (segment (start 150.72868 94.80804) (end 150.72868 94.48804) (width 0.25) (layer B.Cu) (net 6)))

